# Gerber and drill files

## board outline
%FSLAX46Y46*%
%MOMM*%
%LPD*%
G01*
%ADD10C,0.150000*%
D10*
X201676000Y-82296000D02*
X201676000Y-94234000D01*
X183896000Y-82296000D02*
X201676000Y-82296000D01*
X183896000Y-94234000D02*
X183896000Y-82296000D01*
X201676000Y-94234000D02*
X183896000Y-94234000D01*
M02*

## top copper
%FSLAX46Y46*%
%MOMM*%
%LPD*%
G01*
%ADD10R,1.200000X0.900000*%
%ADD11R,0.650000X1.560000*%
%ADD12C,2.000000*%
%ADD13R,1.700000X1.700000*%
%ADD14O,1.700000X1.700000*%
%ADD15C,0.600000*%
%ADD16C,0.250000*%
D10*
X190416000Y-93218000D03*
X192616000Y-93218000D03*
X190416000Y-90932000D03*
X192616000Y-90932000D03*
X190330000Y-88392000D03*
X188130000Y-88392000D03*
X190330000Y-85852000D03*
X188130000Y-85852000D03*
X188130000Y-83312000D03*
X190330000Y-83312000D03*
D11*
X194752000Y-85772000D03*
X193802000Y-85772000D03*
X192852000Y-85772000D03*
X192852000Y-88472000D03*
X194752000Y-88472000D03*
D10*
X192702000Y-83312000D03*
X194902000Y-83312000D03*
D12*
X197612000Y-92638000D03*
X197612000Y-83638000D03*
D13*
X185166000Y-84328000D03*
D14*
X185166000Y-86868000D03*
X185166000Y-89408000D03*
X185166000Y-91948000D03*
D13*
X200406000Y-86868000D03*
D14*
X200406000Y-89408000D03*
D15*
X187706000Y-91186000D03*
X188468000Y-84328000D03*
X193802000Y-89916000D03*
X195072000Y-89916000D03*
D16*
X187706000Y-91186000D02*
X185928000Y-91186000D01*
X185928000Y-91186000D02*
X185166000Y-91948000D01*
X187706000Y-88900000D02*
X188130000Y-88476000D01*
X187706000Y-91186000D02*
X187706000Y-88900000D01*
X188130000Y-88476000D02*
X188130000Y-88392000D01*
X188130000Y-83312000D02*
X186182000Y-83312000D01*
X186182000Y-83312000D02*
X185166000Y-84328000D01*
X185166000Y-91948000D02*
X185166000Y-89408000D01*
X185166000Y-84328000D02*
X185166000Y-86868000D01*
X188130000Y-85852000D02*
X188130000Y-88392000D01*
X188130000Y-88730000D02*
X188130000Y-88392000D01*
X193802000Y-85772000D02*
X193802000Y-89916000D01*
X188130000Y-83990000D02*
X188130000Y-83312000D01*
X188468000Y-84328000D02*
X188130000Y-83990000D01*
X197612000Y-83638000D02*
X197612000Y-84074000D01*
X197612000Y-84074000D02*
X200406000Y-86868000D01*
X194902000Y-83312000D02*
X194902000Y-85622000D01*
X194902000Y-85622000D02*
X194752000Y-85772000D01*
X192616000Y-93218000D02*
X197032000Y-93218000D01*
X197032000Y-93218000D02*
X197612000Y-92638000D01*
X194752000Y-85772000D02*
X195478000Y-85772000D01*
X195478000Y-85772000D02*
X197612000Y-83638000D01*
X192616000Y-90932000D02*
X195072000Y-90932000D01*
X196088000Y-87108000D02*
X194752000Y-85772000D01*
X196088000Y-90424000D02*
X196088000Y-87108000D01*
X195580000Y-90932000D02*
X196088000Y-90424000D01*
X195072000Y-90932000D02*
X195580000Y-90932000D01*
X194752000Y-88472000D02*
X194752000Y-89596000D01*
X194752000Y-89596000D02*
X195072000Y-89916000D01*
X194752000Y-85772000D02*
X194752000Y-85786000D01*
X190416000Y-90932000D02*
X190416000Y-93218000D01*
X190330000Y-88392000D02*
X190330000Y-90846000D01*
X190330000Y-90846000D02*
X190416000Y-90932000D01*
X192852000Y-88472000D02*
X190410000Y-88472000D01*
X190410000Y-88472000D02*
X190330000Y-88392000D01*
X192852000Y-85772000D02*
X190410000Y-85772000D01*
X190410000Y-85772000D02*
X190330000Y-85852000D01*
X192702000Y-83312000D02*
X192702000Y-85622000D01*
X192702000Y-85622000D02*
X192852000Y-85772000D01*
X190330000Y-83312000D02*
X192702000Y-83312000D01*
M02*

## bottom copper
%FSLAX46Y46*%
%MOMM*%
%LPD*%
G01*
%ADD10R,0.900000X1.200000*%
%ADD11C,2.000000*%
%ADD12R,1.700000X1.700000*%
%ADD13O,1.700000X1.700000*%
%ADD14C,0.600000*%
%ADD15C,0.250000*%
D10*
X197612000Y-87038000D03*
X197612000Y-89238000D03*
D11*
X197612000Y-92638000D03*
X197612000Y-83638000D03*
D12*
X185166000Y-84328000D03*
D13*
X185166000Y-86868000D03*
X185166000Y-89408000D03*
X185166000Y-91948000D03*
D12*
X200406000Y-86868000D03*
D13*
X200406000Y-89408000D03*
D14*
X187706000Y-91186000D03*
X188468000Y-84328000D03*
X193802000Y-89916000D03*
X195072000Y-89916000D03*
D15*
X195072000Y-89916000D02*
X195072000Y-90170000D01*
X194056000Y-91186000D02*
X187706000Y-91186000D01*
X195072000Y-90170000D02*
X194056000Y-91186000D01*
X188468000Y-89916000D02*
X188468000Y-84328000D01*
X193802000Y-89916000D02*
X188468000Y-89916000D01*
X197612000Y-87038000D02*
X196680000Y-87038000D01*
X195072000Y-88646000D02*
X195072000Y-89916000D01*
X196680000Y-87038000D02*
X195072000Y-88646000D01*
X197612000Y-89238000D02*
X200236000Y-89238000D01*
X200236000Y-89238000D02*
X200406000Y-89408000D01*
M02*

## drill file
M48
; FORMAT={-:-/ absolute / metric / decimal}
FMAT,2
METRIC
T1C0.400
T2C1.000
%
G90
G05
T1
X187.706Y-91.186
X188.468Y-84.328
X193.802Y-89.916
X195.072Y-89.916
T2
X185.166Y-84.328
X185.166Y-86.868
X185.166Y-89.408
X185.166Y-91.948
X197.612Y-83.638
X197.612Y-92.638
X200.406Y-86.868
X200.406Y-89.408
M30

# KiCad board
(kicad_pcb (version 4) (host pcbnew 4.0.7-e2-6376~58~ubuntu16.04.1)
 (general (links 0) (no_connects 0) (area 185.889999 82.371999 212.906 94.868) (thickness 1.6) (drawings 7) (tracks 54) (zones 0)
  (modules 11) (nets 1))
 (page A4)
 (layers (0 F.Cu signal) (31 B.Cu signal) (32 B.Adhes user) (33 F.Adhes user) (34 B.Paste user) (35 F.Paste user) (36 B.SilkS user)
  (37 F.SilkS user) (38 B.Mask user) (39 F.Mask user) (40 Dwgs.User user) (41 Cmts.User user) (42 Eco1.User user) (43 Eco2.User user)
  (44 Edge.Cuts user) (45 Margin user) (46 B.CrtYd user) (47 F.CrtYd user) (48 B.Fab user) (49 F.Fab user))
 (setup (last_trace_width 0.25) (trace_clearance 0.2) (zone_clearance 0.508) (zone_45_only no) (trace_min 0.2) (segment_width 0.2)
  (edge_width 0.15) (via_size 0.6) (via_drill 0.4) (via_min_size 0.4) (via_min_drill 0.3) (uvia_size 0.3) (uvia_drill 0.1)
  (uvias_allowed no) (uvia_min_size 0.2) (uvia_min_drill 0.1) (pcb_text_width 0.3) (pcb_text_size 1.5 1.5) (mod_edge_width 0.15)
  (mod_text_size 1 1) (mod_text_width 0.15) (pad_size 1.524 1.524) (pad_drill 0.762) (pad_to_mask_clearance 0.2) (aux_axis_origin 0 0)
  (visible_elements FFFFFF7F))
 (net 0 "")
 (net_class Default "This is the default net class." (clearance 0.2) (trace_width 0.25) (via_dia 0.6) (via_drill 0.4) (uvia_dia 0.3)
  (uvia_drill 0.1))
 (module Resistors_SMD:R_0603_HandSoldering (layer B.Cu) (at 197.612 88.138 270)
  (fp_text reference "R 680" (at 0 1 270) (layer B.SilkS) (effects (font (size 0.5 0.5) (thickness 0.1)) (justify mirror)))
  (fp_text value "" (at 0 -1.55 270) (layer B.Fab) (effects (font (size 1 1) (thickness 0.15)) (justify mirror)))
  (pad 1 smd rect (at -1.1 0 270) (size 1.2 0.9) (layers B.Cu B.Paste B.Mask))
  (pad 2 smd rect (at 1.1 0 270) (size 1.2 0.9) (layers B.Cu B.Paste B.Mask)))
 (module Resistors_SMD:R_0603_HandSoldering (layer F.Cu) (at 191.516 93.218)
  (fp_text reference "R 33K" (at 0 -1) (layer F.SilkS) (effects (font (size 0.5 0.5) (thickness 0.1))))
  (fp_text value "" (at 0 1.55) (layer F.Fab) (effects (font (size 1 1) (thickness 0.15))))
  (pad 1 smd rect (at -1.1 0) (size 1.2 0.9) (layers F.Cu F.Paste F.Mask))
  (pad 2 smd rect (at 1.1 0) (size 1.2 0.9) (layers F.Cu F.Paste F.Mask)))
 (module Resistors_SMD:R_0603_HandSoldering (layer F.Cu) (at 191.516 90.932)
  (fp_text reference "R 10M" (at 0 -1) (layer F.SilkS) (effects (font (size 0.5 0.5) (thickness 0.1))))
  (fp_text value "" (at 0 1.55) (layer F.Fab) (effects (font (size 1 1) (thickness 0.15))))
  (pad 1 smd rect (at -1.1 0) (size 1.2 0.9) (layers F.Cu F.Paste F.Mask))
  (pad 2 smd rect (at 1.1 0) (size 1.2 0.9) (layers F.Cu F.Paste F.Mask)))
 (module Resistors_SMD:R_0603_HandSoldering (layer F.Cu) (at 189.23 88.392 180)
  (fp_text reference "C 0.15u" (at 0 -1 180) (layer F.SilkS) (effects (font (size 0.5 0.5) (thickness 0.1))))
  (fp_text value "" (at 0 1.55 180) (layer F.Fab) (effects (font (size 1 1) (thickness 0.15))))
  (pad 1 smd rect (at -1.1 0 180) (size 1.2 0.9) (layers F.Cu F.Paste F.Mask))
  (pad 2 smd rect (at 1.1 0 180) (size 1.2 0.9) (layers F.Cu F.Paste F.Mask)))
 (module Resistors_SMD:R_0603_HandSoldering (layer F.Cu) (at 189.23 85.852 180)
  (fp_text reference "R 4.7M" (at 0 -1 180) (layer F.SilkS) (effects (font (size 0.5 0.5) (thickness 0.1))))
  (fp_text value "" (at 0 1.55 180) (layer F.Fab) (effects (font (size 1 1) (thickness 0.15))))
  (pad 1 smd rect (at -1.1 0 180) (size 1.2 0.9) (layers F.Cu F.Paste F.Mask))
  (pad 2 smd rect (at 1.1 0 180) (size 1.2 0.9) (layers F.Cu F.Paste F.Mask)))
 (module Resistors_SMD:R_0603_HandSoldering (layer F.Cu) (at 189.23 83.312)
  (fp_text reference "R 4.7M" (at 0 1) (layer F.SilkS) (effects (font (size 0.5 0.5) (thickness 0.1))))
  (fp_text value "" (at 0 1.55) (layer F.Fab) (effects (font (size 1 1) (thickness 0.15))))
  (pad 1 smd rect (at -1.1 0) (size 1.2 0.9) (layers F.Cu F.Paste F.Mask))
  (pad 2 smd rect (at 1.1 0) (size 1.2 0.9) (layers F.Cu F.Paste F.Mask)))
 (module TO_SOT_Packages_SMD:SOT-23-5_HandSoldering (layer F.Cu) (at 193.802 87.122 270)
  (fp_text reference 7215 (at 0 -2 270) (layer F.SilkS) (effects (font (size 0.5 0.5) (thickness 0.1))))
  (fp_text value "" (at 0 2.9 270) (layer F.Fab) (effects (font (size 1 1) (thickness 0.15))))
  (pad 1 smd rect (at -1.35 -0.95 270) (size 1.56 0.65) (layers F.Cu F.Paste F.Mask))
  (pad 2 smd rect (at -1.35 0 270) (size 1.56 0.65) (layers F.Cu F.Paste F.Mask))
  (pad 3 smd rect (at -1.35 0.95 270) (size 1.56 0.65) (layers F.Cu F.Paste F.Mask))
  (pad 4 smd rect (at 1.35 0.95 270) (size 1.56 0.65) (layers F.Cu F.Paste F.Mask))
  (pad 5 smd rect (at 1.35 -0.95 270) (size 1.56 0.65) (layers F.Cu F.Paste F.Mask)))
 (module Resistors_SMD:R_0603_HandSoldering (layer F.Cu) (at 193.802 83.312)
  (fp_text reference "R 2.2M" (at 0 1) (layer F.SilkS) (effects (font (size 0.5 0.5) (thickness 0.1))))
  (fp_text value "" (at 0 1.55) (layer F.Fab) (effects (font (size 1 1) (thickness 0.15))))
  (pad 1 smd rect (at -1.1 0) (size 1.2 0.9) (layers F.Cu F.Paste F.Mask))
  (pad 2 smd rect (at 1.1 0) (size 1.2 0.9) (layers F.Cu F.Paste F.Mask)))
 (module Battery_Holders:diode (layer F.Cu) (at 197.612 88.138 90)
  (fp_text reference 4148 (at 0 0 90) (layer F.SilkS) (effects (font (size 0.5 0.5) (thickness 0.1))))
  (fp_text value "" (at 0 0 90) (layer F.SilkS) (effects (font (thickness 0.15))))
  (pad 1 thru_hole circle (at -4.5 0 90) (size 2 2) (drill 1) (layers *.Cu *.Mask))
  (pad 2 thru_hole circle (at 4.5 0 90) (size 2 2) (drill 1) (layers *.Cu *.Mask)))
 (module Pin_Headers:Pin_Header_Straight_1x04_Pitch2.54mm (layer F.Cu) (at 185.166 84.328)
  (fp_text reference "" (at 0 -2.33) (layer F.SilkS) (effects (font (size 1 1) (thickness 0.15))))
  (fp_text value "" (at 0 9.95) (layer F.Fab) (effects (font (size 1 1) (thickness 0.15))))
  (pad 1 thru_hole rect (at 0 0) (size 1.7 1.7) (drill 1) (layers *.Cu *.Mask))
  (pad 2 thru_hole oval (at 0 2.54) (size 1.7 1.7) (drill 1) (layers *.Cu *.Mask))
  (pad 3 thru_hole oval (at 0 5.08) (size 1.7 1.7) (drill 1) (layers *.Cu *.Mask))
  (pad 4 thru_hole oval (at 0 7.62) (size 1.7 1.7) (drill 1) (layers *.Cu *.Mask)))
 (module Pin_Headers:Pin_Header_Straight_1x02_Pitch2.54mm (layer F.Cu) (at 200.406 86.868)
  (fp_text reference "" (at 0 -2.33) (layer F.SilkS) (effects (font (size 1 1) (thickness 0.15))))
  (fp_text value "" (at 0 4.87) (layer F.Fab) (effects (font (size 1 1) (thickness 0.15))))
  (pad 1 thru_hole rect (at 0 0) (size 1.7 1.7) (drill 1) (layers *.Cu *.Mask))
  (pad 2 thru_hole oval (at 0 2.54) (size 1.7 1.7) (drill 1) (layers *.Cu *.Mask)))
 (gr_line (start 201.676 82.296) (end 201.676 94.234) (angle 90) (layer Edge.Cuts) (width 0.15))
 (gr_line (start 183.896 82.296) (end 201.676 82.296) (angle 90) (layer Edge.Cuts) (width 0.15))
 (gr_line (start 183.896 94.234) (end 183.896 82.296) (angle 90) (layer Edge.Cuts) (width 0.15))
 (gr_line (start 201.676 94.234) (end 183.896 94.234) (angle 90) (layer Edge.Cuts) (width 0.15))
 (segment (start 187.706 91.186) (end 185.928 91.186) (width 0.25) (layer F.Cu) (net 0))
 (segment (start 185.928 91.186) (end 185.166 91.948) (width 0.25) (layer F.Cu) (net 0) (status 800000))
 (segment (start 195.072 89.916) (end 195.072 90.17) (width 0.25) (layer B.Cu) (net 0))
 (segment (start 187.706 88.9) (end 188.13 88.476) (width 0.25) (layer F.Cu) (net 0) (status 800000))
 (segment (start 187.706 91.186) (end 187.706 88.9) (width 0.25) (layer F.Cu) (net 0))
 (via (at 187.706 91.186) (size 0.6) (drill 0.4) (layers F.Cu B.Cu) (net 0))
 (segment (start 194.056 91.186) (end 187.706 91.186) (width 0.25) (layer B.Cu) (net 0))
 (segment (start 195.072 90.17) (end 194.056 91.186) (width 0.25) (layer B.Cu) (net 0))
 (segment (start 188.13 88.476) (end 188.13 88.392) (width 0.25) (layer F.Cu) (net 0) (status C00000))
 (segment (start 188.13 83.312) (end 186.182 83.312) (width 0.25) (layer F.Cu) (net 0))
 (segment (start 186.182 83.312) (end 185.166 84.328) (width 0.25) (layer F.Cu) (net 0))
 (segment (start 185.166 91.948) (end 185.166 89.408) (width 0.25) (layer F.Cu) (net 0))
 (segment (start 185.166 84.328) (end 185.166 86.868) (width 0.25) (layer F.Cu) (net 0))
 (segment (start 188.13 85.852) (end 188.13 88.392) (width 0.25) (layer F.Cu) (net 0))
 (segment (start 188.13 88.73) (end 188.13 88.392) (width 0.25) (layer F.Cu) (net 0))
 (segment (start 193.802 85.772) (end 193.802 89.916) (width 0.25) (layer F.Cu) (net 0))
 (segment (start 188.13 83.99) (end 188.13 83.312) (width 0.25) (layer F.Cu) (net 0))
 (segment (start 188.468 84.328) (end 188.13 83.99) (width 0.25) (layer F.Cu) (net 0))
 (via (at 188.468 84.328) (size 0.6) (drill 0.4) (layers F.Cu B.Cu) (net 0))
 (segment (start 188.468 89.916) (end 188.468 84.328) (width 0.25) (layer B.Cu) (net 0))
 (segment (start 193.802 89.916) (end 188.468 89.916) (width 0.25) (layer B.Cu) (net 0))
 (via (at 193.802 89.916) (size 0.6) (drill 0.4) (layers F.Cu B.Cu) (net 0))
 (segment (start 197.612 87.038) (end 196.68 87.038) (width 0.25) (layer B.Cu) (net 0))
 (segment (start 195.072 88.646) (end 195.072 89.916) (width 0.25) (layer B.Cu) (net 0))
 (segment (start 196.68 87.038) (end 195.072 88.646) (width 0.25) (layer B.Cu) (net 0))
 (segment (start 197.612 89.238) (end 200.236 89.238) (width 0.25) (layer B.Cu) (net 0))
 (segment (start 200.236 89.238) (end 200.406 89.408) (width 0.25) (layer B.Cu) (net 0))
 (segment (start 197.612 83.638) (end 197.612 84.074) (width 0.25) (layer F.Cu) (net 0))
 (segment (start 197.612 84.074) (end 200.406 86.868) (width 0.25) (layer F.Cu) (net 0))
 (segment (start 194.902 83.312) (end 194.902 85.622) (width 0.25) (layer F.Cu) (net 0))
 (segment (start 194.902 85.622) (end 194.752 85.772) (width 0.25) (layer F.Cu) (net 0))
 (segment (start 192.616 93.218) (end 197.032 93.218) (width 0.25) (layer F.Cu) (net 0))
 (segment (start 197.032 93.218) (end 197.612 92.638) (width 0.25) (layer F.Cu) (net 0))
 (segment (start 194.752 85.772) (end 195.478 85.772) (width 0.25) (layer F.Cu) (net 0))
 (segment (start 195.478 85.772) (end 197.612 83.638) (width 0.25) (layer F.Cu) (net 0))
 (segment (start 192.616 90.932) (end 195.072 90.932) (width 0.25) (layer F.Cu) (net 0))
 (segment (start 196.088 87.108) (end 194.752 85.772) (width 0.25) (layer F.Cu) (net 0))
 (segment (start 196.088 90.424) (end 196.088 87.108) (width 0.25) (layer F.Cu) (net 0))
 (segment (start 195.58 90.932) (end 196.088 90.424) (width 0.25) (layer F.Cu) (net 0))
 (segment (start 195.072 90.932) (end 195.58 90.932) (width 0.25) (layer F.Cu) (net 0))
 (segment (start 194.752 88.472) (end 194.752 89.596) (width 0.25) (layer F.Cu) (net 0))
 (via (at 195.072 89.916) (size 0.6) (drill 0.4) (layers F.Cu B.Cu) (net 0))
 (segment (start 194.752 89.596) (end 195.072 89.916) (width 0.25) (layer F.Cu) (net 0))
 (segment (start 194.752 85.772) (end 194.752 85.786) (width 0.25) (layer F.Cu) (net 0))
 (segment (start 190.416 90.932) (end 190.416 93.218) (width 0.25) (layer F.Cu) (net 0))
 (segment (start 190.33 88.392) (end 190.33 90.846) (width 0.25) (layer F.Cu) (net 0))
 (segment (start 190.33 90.846) (end 190.416 90.932) (width 0.25) (layer F.Cu) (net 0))
 (segment (start 192.852 88.472) (end 190.41 88.472) (width 0.25) (layer F.Cu) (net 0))
 (segment (start 190.41 88.472) (end 190.33 88.392) (width 0.25) (layer F.Cu) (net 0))
 (segment (start 192.852 85.772) (end 190.41 85.772) (width 0.25) (layer F.Cu) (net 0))
 (segment (start 190.41 85.772) (end 190.33 85.852) (width 0.25) (layer F.Cu) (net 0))
 (segment (start 192.702 83.312) (end 192.702 85.622) (width 0.25) (layer F.Cu) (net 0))
 (segment (start 192.702 85.622) (end 192.852 85.772) (width 0.25) (layer F.Cu) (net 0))
 (segment (start 190.33 83.312) (end 192.702 83.312) (width 0.25) (layer F.Cu) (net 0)))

